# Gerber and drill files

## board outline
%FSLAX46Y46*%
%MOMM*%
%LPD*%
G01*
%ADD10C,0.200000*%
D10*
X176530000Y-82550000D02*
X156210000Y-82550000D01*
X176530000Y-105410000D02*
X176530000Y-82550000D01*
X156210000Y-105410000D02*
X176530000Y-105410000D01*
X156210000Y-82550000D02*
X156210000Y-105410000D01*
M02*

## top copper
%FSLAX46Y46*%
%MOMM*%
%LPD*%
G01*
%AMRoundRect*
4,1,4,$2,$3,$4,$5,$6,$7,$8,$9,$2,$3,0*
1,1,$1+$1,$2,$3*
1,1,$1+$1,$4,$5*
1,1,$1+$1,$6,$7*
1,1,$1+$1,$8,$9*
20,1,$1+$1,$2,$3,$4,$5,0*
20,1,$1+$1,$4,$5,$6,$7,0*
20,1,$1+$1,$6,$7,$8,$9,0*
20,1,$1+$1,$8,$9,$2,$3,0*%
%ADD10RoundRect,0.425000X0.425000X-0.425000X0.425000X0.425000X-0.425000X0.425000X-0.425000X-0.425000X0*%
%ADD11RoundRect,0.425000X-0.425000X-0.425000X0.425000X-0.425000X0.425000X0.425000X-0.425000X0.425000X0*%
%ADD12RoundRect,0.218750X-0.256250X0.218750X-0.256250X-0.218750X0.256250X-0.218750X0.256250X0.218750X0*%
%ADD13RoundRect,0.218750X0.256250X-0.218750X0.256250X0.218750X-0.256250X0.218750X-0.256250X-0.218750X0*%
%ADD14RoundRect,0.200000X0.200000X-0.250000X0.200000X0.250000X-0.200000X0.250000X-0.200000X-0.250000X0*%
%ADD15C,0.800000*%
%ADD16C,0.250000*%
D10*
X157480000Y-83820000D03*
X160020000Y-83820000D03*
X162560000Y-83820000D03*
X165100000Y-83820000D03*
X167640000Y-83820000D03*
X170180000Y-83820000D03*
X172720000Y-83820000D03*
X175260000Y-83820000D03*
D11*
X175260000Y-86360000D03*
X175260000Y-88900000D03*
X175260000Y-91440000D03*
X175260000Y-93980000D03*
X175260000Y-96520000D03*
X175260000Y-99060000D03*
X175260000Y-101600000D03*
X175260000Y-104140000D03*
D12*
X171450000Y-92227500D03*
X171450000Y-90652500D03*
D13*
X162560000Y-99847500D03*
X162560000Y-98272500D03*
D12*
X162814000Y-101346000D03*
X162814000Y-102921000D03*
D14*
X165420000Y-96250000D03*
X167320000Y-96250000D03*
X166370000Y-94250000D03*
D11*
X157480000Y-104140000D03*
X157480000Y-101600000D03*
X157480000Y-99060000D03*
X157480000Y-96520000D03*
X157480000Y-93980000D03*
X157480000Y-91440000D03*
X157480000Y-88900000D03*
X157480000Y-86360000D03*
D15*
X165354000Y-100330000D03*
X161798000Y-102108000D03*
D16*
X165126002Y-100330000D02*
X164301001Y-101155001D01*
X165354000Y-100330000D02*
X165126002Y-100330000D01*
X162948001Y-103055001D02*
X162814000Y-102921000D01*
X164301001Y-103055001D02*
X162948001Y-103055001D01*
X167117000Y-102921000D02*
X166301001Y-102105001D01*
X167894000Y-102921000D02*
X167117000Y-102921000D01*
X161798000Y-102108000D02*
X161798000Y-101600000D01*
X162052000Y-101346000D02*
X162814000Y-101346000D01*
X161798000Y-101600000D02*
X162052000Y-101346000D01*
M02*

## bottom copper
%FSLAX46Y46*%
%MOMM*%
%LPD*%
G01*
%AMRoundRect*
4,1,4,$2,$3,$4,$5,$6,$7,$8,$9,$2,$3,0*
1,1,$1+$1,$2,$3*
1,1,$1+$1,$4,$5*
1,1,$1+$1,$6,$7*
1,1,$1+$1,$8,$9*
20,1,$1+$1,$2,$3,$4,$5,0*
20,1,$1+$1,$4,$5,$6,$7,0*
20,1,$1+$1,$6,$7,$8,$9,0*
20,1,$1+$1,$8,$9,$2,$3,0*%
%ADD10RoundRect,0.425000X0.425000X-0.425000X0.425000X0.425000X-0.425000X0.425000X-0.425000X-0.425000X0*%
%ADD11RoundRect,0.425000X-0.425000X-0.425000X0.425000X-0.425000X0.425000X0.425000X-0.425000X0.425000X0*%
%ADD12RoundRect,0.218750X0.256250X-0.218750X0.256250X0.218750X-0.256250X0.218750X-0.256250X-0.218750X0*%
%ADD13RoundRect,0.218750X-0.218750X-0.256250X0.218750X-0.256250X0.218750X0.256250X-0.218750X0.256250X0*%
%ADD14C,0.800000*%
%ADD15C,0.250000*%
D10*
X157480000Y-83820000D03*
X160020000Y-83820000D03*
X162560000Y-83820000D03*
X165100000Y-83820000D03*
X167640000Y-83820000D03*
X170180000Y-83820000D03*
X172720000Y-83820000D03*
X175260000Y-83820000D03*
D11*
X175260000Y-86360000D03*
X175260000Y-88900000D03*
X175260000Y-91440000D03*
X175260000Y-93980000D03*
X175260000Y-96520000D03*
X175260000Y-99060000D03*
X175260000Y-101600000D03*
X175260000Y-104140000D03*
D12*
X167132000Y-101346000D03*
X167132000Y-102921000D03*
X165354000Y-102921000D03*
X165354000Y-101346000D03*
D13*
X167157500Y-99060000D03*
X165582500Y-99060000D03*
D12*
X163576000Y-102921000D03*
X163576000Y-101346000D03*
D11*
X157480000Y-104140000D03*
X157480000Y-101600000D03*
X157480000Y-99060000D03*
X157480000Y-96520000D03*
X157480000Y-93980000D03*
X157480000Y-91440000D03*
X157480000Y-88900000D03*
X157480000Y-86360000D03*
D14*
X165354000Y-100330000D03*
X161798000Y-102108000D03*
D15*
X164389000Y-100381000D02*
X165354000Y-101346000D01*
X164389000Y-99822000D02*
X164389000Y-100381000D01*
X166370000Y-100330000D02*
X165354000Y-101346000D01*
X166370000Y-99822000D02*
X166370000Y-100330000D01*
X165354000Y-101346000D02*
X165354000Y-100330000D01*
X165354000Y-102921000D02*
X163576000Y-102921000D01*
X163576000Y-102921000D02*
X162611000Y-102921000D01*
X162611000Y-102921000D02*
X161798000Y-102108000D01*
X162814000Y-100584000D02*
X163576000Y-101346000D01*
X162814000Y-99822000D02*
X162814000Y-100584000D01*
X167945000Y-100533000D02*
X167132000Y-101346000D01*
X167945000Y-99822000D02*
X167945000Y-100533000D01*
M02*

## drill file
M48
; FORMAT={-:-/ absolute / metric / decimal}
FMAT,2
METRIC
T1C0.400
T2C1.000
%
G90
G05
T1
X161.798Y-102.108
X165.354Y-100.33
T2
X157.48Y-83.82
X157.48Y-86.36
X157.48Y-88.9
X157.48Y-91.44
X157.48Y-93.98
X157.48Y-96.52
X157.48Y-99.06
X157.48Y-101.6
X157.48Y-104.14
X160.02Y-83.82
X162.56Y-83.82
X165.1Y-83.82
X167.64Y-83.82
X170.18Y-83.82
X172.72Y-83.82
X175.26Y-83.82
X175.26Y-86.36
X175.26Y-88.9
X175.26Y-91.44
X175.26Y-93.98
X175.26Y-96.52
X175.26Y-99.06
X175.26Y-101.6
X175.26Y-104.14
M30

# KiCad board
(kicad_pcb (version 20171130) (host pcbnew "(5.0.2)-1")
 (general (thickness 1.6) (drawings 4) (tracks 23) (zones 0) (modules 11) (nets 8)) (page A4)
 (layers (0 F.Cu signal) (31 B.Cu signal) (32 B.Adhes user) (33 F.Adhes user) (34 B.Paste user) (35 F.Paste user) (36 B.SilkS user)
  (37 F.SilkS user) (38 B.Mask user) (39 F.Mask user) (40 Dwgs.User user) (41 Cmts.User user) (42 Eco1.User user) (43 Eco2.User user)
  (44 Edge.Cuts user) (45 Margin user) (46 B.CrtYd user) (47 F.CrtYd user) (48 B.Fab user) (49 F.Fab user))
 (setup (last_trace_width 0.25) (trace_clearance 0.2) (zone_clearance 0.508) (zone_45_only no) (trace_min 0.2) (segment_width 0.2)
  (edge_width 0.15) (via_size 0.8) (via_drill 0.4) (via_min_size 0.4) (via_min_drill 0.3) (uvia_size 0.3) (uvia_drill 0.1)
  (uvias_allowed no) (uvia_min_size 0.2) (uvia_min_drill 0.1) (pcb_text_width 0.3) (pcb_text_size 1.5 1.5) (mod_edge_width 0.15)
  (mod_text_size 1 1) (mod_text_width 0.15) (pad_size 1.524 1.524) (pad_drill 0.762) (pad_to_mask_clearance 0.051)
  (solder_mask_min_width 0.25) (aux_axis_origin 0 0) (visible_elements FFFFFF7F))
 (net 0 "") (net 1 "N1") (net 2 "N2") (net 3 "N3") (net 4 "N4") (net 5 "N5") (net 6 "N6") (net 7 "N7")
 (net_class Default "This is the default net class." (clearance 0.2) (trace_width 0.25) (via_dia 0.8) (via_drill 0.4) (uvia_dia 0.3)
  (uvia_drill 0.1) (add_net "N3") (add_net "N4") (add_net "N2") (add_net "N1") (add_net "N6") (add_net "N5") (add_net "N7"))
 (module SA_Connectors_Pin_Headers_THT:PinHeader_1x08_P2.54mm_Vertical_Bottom (layer F.Cu) (at 157.48 83.82 90)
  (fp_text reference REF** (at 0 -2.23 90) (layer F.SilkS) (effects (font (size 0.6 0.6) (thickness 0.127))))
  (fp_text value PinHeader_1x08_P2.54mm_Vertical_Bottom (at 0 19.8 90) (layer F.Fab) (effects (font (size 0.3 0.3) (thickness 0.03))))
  (pad 1 thru_hole roundrect (at 0 0 90) (size 1.7 1.7) (drill 1) (layers *.Cu *.Mask) (roundrect_rratio 0.25))
  (pad 2 thru_hole roundrect (at 0 2.54 90) (size 1.7 1.7) (drill 1) (layers *.Cu *.Mask) (roundrect_rratio 0.25))
  (pad 3 thru_hole roundrect (at 0 5.08 90) (size 1.7 1.7) (drill 1) (layers *.Cu *.Mask) (roundrect_rratio 0.25))
  (pad 4 thru_hole roundrect (at 0 7.62 90) (size 1.7 1.7) (drill 1) (layers *.Cu *.Mask) (roundrect_rratio 0.25))
  (pad 5 thru_hole roundrect (at 0 10.16 90) (size 1.7 1.7) (drill 1) (layers *.Cu *.Mask) (roundrect_rratio 0.25))
  (pad 6 thru_hole roundrect (at 0 12.7 90) (size 1.7 1.7) (drill 1) (layers *.Cu *.Mask) (roundrect_rratio 0.25))
  (pad 7 thru_hole roundrect (at 0 15.24 90) (size 1.7 1.7) (drill 1) (layers *.Cu *.Mask) (roundrect_rratio 0.25))
  (pad 8 thru_hole roundrect (at 0 17.78 90) (size 1.7 1.7) (drill 1) (layers *.Cu *.Mask) (roundrect_rratio 0.25)))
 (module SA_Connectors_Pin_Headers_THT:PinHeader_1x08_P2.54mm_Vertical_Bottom (layer F.Cu) (at 175.26 86.36)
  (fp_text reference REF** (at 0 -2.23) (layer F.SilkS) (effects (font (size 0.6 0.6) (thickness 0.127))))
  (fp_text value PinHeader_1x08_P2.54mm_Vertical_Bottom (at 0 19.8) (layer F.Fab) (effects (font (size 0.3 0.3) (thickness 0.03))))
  (pad 1 thru_hole roundrect (at 0 0) (size 1.7 1.7) (drill 1) (layers *.Cu *.Mask) (roundrect_rratio 0.25))
  (pad 2 thru_hole roundrect (at 0 2.54) (size 1.7 1.7) (drill 1) (layers *.Cu *.Mask) (roundrect_rratio 0.25))
  (pad 3 thru_hole roundrect (at 0 5.08) (size 1.7 1.7) (drill 1) (layers *.Cu *.Mask) (roundrect_rratio 0.25))
  (pad 4 thru_hole roundrect (at 0 7.62) (size 1.7 1.7) (drill 1) (layers *.Cu *.Mask) (roundrect_rratio 0.25))
  (pad 5 thru_hole roundrect (at 0 10.16) (size 1.7 1.7) (drill 1) (layers *.Cu *.Mask) (roundrect_rratio 0.25))
  (pad 6 thru_hole roundrect (at 0 12.7) (size 1.7 1.7) (drill 1) (layers *.Cu *.Mask) (roundrect_rratio 0.25))
  (pad 7 thru_hole roundrect (at 0 15.24) (size 1.7 1.7) (drill 1) (layers *.Cu *.Mask) (roundrect_rratio 0.25))
  (pad 8 thru_hole roundrect (at 0 17.78) (size 1.7 1.7) (drill 1) (layers *.Cu *.Mask) (roundrect_rratio 0.25)))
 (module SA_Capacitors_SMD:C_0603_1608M (layer F.Cu) (at 171.45 91.44 270)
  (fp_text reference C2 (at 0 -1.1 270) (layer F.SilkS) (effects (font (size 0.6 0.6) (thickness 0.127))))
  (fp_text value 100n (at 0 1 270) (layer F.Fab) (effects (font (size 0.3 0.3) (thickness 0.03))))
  (pad 2 smd roundrect (at 0.7875 0 270) (size 0.875 0.95) (layers F.Cu F.Paste F.Mask) (roundrect_rratio 0.25) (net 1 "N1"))
  (pad 1 smd roundrect (at -0.7875 0 270) (size 0.875 0.95) (layers F.Cu F.Paste F.Mask) (roundrect_rratio 0.25) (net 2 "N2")))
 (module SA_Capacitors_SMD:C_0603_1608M (layer F.Cu) (at 162.56 99.06 90)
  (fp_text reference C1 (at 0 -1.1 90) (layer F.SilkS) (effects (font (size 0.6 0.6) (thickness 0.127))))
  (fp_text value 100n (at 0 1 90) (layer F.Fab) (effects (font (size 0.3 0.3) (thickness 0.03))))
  (pad 1 smd roundrect (at -0.7875 0 90) (size 0.875 0.95) (layers F.Cu F.Paste F.Mask) (roundrect_rratio 0.25) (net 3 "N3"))
  (pad 2 smd roundrect (at 0.7875 0 90) (size 0.875 0.95) (layers F.Cu F.Paste F.Mask) (roundrect_rratio 0.25) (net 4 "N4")))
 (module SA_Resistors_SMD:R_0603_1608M (layer F.Cu) (at 162.814 102.1335 270)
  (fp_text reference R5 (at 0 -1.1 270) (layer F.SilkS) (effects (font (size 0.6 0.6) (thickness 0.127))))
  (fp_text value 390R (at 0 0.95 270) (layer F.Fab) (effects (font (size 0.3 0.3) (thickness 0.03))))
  (pad 1 smd roundrect (at -0.7875 0 270) (size 0.875 0.95) (layers F.Cu F.Paste F.Mask) (roundrect_rratio 0.25) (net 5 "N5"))
  (pad 2 smd roundrect (at 0.7875 0 270) (size 0.875 0.95) (layers F.Cu F.Paste F.Mask) (roundrect_rratio 0.25) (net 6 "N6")))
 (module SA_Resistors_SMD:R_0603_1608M (layer B.Cu) (at 167.132 102.1335 90)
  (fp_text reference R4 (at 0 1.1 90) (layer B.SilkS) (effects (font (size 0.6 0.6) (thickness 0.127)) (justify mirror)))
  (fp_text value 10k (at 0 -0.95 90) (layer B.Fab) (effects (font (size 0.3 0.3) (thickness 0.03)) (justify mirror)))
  (pad 2 smd roundrect (at 0.7875 0 90) (size 0.875 0.95) (layers B.Cu B.Paste B.Mask) (roundrect_rratio 0.25) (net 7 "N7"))
  (pad 1 smd roundrect (at -0.7875 0 90) (size 0.875 0.95) (layers B.Cu B.Paste B.Mask) (roundrect_rratio 0.25) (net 2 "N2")))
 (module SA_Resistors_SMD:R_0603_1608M (layer B.Cu) (at 165.354 102.1335 90)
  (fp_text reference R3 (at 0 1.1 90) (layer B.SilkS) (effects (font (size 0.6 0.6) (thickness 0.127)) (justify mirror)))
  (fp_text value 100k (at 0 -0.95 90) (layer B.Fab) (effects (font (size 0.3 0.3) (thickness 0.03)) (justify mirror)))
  (pad 1 smd roundrect (at -0.7875 0 90) (size 0.875 0.95) (layers B.Cu B.Paste B.Mask) (roundrect_rratio 0.25) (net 5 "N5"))
  (pad 2 smd roundrect (at 0.7875 0 90) (size 0.875 0.95) (layers B.Cu B.Paste B.Mask) (roundrect_rratio 0.25) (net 4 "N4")))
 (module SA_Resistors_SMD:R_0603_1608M (layer B.Cu) (at 166.37 99.06)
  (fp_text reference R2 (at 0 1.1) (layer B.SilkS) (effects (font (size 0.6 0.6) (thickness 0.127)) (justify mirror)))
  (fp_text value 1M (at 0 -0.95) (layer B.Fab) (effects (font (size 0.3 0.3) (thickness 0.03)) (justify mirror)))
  (pad 2 smd roundrect (at 0.7875 0) (size 0.875 0.95) (layers B.Cu B.Paste B.Mask) (roundrect_rratio 0.25) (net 7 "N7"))
  (pad 1 smd roundrect (at -0.7875 0) (size 0.875 0.95) (layers B.Cu B.Paste B.Mask) (roundrect_rratio 0.25) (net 4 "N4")))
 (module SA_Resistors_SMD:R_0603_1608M (layer B.Cu) (at 163.576 102.1335 90)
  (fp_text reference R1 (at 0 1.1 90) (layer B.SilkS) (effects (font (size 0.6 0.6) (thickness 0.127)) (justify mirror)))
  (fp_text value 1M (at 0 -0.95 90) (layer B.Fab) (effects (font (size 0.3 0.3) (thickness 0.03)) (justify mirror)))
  (pad 1 smd roundrect (at -0.7875 0 90) (size 0.875 0.95) (layers B.Cu B.Paste B.Mask) (roundrect_rratio 0.25) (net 5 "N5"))
  (pad 2 smd roundrect (at 0.7875 0 90) (size 0.875 0.95) (layers B.Cu B.Paste B.Mask) (roundrect_rratio 0.25) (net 3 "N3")))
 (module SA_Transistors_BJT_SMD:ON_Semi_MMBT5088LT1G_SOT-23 (layer F.Cu) (at 166.37 95.25 90)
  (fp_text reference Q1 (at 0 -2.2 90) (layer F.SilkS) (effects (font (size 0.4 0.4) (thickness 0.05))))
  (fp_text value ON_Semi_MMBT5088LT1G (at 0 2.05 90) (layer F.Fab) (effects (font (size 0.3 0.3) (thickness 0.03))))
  (pad 1 smd roundrect (at -1 -0.95 90) (size 0.9 0.8) (layers F.Cu F.Paste F.Mask) (roundrect_rratio 0.25) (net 4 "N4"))
  (pad 2 smd roundrect (at -1 0.95 90) (size 0.9 0.8) (layers F.Cu F.Paste F.Mask) (roundrect_rratio 0.25) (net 6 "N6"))
  (pad 3 smd roundrect (at 1 0 90) (size 0.9 0.8) (layers F.Cu F.Paste F.Mask) (roundrect_rratio 0.25) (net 2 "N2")))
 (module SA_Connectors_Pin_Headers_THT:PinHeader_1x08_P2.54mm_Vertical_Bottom (layer F.Cu) (at 157.48 86.36)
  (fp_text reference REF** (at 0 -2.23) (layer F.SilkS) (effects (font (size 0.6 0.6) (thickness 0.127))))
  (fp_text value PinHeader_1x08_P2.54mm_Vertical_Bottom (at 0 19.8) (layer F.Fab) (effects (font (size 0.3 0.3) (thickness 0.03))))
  (pad 8 thru_hole roundrect (at 0 17.78) (size 1.7 1.7) (drill 1) (layers *.Cu *.Mask) (roundrect_rratio 0.25))
  (pad 7 thru_hole roundrect (at 0 15.24) (size 1.7 1.7) (drill 1) (layers *.Cu *.Mask) (roundrect_rratio 0.25))
  (pad 6 thru_hole roundrect (at 0 12.7) (size 1.7 1.7) (drill 1) (layers *.Cu *.Mask) (roundrect_rratio 0.25))
  (pad 5 thru_hole roundrect (at 0 10.16) (size 1.7 1.7) (drill 1) (layers *.Cu *.Mask) (roundrect_rratio 0.25))
  (pad 4 thru_hole roundrect (at 0 7.62) (size 1.7 1.7) (drill 1) (layers *.Cu *.Mask) (roundrect_rratio 0.25))
  (pad 3 thru_hole roundrect (at 0 5.08) (size 1.7 1.7) (drill 1) (layers *.Cu *.Mask) (roundrect_rratio 0.25))
  (pad 2 thru_hole roundrect (at 0 2.54) (size 1.7 1.7) (drill 1) (layers *.Cu *.Mask) (roundrect_rratio 0.25))
  (pad 1 thru_hole roundrect (at 0 0) (size 1.7 1.7) (drill 1) (layers *.Cu *.Mask) (roundrect_rratio 0.25)))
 (gr_line (start 176.53 82.55) (end 156.21 82.55) (layer Edge.Cuts) (width 0.2))
 (gr_line (start 176.53 105.41) (end 176.53 82.55) (layer Edge.Cuts) (width 0.2))
 (gr_line (start 156.21 105.41) (end 176.53 105.41) (layer Edge.Cuts) (width 0.2))
 (gr_line (start 156.21 82.55) (end 156.21 105.41) (layer Edge.Cuts) (width 0.2))
 (segment (start 164.389 100.381) (end 165.354 101.346) (width 0.25) (layer B.Cu) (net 4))
 (segment (start 164.389 99.822) (end 164.389 100.381) (width 0.25) (layer B.Cu) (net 4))
 (segment (start 166.37 100.33) (end 165.354 101.346) (width 0.25) (layer B.Cu) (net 4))
 (segment (start 166.37 99.822) (end 166.37 100.33) (width 0.25) (layer B.Cu) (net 4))
 (via (at 165.354 100.33) (size 0.8) (drill 0.4) (layers F.Cu B.Cu) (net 4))
 (segment (start 165.354 101.346) (end 165.354 100.33) (width 0.25) (layer B.Cu) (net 4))
 (segment (start 165.126002 100.33) (end 164.301001 101.155001) (width 0.25) (layer F.Cu) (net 4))
 (segment (start 165.354 100.33) (end 165.126002 100.33) (width 0.25) (layer F.Cu) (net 4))
 (segment (start 162.948001 103.055001) (end 162.814 102.921) (width 0.25) (layer F.Cu) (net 6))
 (segment (start 164.301001 103.055001) (end 162.948001 103.055001) (width 0.25) (layer F.Cu) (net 6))
 (segment (start 167.117 102.921) (end 166.301001 102.105001) (width 0.25) (layer F.Cu) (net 2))
 (segment (start 167.894 102.921) (end 167.117 102.921) (width 0.25) (layer F.Cu) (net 2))
 (segment (start 165.354 102.921) (end 163.576 102.921) (width 0.25) (layer B.Cu) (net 5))
 (via (at 161.798 102.108) (size 0.8) (drill 0.4) (layers F.Cu B.Cu) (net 5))
 (segment (start 163.576 102.921) (end 162.611 102.921) (width 0.25) (layer B.Cu) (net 5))
 (segment (start 162.611 102.921) (end 161.798 102.108) (width 0.25) (layer B.Cu) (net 5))
 (segment (start 161.798 102.108) (end 161.798 101.6) (width 0.25) (layer F.Cu) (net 5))
 (segment (start 162.052 101.346) (end 162.814 101.346) (width 0.25) (layer F.Cu) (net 5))
 (segment (start 161.798 101.6) (end 162.052 101.346) (width 0.25) (layer F.Cu) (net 5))
 (segment (start 162.814 100.584) (end 163.576 101.346) (width 0.25) (layer B.Cu) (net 3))
 (segment (start 162.814 99.822) (end 162.814 100.584) (width 0.25) (layer B.Cu) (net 3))
 (segment (start 167.945 100.533) (end 167.132 101.346) (width 0.25) (layer B.Cu) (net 7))
 (segment (start 167.945 99.822) (end 167.945 100.533) (width 0.25) (layer B.Cu) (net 7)))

